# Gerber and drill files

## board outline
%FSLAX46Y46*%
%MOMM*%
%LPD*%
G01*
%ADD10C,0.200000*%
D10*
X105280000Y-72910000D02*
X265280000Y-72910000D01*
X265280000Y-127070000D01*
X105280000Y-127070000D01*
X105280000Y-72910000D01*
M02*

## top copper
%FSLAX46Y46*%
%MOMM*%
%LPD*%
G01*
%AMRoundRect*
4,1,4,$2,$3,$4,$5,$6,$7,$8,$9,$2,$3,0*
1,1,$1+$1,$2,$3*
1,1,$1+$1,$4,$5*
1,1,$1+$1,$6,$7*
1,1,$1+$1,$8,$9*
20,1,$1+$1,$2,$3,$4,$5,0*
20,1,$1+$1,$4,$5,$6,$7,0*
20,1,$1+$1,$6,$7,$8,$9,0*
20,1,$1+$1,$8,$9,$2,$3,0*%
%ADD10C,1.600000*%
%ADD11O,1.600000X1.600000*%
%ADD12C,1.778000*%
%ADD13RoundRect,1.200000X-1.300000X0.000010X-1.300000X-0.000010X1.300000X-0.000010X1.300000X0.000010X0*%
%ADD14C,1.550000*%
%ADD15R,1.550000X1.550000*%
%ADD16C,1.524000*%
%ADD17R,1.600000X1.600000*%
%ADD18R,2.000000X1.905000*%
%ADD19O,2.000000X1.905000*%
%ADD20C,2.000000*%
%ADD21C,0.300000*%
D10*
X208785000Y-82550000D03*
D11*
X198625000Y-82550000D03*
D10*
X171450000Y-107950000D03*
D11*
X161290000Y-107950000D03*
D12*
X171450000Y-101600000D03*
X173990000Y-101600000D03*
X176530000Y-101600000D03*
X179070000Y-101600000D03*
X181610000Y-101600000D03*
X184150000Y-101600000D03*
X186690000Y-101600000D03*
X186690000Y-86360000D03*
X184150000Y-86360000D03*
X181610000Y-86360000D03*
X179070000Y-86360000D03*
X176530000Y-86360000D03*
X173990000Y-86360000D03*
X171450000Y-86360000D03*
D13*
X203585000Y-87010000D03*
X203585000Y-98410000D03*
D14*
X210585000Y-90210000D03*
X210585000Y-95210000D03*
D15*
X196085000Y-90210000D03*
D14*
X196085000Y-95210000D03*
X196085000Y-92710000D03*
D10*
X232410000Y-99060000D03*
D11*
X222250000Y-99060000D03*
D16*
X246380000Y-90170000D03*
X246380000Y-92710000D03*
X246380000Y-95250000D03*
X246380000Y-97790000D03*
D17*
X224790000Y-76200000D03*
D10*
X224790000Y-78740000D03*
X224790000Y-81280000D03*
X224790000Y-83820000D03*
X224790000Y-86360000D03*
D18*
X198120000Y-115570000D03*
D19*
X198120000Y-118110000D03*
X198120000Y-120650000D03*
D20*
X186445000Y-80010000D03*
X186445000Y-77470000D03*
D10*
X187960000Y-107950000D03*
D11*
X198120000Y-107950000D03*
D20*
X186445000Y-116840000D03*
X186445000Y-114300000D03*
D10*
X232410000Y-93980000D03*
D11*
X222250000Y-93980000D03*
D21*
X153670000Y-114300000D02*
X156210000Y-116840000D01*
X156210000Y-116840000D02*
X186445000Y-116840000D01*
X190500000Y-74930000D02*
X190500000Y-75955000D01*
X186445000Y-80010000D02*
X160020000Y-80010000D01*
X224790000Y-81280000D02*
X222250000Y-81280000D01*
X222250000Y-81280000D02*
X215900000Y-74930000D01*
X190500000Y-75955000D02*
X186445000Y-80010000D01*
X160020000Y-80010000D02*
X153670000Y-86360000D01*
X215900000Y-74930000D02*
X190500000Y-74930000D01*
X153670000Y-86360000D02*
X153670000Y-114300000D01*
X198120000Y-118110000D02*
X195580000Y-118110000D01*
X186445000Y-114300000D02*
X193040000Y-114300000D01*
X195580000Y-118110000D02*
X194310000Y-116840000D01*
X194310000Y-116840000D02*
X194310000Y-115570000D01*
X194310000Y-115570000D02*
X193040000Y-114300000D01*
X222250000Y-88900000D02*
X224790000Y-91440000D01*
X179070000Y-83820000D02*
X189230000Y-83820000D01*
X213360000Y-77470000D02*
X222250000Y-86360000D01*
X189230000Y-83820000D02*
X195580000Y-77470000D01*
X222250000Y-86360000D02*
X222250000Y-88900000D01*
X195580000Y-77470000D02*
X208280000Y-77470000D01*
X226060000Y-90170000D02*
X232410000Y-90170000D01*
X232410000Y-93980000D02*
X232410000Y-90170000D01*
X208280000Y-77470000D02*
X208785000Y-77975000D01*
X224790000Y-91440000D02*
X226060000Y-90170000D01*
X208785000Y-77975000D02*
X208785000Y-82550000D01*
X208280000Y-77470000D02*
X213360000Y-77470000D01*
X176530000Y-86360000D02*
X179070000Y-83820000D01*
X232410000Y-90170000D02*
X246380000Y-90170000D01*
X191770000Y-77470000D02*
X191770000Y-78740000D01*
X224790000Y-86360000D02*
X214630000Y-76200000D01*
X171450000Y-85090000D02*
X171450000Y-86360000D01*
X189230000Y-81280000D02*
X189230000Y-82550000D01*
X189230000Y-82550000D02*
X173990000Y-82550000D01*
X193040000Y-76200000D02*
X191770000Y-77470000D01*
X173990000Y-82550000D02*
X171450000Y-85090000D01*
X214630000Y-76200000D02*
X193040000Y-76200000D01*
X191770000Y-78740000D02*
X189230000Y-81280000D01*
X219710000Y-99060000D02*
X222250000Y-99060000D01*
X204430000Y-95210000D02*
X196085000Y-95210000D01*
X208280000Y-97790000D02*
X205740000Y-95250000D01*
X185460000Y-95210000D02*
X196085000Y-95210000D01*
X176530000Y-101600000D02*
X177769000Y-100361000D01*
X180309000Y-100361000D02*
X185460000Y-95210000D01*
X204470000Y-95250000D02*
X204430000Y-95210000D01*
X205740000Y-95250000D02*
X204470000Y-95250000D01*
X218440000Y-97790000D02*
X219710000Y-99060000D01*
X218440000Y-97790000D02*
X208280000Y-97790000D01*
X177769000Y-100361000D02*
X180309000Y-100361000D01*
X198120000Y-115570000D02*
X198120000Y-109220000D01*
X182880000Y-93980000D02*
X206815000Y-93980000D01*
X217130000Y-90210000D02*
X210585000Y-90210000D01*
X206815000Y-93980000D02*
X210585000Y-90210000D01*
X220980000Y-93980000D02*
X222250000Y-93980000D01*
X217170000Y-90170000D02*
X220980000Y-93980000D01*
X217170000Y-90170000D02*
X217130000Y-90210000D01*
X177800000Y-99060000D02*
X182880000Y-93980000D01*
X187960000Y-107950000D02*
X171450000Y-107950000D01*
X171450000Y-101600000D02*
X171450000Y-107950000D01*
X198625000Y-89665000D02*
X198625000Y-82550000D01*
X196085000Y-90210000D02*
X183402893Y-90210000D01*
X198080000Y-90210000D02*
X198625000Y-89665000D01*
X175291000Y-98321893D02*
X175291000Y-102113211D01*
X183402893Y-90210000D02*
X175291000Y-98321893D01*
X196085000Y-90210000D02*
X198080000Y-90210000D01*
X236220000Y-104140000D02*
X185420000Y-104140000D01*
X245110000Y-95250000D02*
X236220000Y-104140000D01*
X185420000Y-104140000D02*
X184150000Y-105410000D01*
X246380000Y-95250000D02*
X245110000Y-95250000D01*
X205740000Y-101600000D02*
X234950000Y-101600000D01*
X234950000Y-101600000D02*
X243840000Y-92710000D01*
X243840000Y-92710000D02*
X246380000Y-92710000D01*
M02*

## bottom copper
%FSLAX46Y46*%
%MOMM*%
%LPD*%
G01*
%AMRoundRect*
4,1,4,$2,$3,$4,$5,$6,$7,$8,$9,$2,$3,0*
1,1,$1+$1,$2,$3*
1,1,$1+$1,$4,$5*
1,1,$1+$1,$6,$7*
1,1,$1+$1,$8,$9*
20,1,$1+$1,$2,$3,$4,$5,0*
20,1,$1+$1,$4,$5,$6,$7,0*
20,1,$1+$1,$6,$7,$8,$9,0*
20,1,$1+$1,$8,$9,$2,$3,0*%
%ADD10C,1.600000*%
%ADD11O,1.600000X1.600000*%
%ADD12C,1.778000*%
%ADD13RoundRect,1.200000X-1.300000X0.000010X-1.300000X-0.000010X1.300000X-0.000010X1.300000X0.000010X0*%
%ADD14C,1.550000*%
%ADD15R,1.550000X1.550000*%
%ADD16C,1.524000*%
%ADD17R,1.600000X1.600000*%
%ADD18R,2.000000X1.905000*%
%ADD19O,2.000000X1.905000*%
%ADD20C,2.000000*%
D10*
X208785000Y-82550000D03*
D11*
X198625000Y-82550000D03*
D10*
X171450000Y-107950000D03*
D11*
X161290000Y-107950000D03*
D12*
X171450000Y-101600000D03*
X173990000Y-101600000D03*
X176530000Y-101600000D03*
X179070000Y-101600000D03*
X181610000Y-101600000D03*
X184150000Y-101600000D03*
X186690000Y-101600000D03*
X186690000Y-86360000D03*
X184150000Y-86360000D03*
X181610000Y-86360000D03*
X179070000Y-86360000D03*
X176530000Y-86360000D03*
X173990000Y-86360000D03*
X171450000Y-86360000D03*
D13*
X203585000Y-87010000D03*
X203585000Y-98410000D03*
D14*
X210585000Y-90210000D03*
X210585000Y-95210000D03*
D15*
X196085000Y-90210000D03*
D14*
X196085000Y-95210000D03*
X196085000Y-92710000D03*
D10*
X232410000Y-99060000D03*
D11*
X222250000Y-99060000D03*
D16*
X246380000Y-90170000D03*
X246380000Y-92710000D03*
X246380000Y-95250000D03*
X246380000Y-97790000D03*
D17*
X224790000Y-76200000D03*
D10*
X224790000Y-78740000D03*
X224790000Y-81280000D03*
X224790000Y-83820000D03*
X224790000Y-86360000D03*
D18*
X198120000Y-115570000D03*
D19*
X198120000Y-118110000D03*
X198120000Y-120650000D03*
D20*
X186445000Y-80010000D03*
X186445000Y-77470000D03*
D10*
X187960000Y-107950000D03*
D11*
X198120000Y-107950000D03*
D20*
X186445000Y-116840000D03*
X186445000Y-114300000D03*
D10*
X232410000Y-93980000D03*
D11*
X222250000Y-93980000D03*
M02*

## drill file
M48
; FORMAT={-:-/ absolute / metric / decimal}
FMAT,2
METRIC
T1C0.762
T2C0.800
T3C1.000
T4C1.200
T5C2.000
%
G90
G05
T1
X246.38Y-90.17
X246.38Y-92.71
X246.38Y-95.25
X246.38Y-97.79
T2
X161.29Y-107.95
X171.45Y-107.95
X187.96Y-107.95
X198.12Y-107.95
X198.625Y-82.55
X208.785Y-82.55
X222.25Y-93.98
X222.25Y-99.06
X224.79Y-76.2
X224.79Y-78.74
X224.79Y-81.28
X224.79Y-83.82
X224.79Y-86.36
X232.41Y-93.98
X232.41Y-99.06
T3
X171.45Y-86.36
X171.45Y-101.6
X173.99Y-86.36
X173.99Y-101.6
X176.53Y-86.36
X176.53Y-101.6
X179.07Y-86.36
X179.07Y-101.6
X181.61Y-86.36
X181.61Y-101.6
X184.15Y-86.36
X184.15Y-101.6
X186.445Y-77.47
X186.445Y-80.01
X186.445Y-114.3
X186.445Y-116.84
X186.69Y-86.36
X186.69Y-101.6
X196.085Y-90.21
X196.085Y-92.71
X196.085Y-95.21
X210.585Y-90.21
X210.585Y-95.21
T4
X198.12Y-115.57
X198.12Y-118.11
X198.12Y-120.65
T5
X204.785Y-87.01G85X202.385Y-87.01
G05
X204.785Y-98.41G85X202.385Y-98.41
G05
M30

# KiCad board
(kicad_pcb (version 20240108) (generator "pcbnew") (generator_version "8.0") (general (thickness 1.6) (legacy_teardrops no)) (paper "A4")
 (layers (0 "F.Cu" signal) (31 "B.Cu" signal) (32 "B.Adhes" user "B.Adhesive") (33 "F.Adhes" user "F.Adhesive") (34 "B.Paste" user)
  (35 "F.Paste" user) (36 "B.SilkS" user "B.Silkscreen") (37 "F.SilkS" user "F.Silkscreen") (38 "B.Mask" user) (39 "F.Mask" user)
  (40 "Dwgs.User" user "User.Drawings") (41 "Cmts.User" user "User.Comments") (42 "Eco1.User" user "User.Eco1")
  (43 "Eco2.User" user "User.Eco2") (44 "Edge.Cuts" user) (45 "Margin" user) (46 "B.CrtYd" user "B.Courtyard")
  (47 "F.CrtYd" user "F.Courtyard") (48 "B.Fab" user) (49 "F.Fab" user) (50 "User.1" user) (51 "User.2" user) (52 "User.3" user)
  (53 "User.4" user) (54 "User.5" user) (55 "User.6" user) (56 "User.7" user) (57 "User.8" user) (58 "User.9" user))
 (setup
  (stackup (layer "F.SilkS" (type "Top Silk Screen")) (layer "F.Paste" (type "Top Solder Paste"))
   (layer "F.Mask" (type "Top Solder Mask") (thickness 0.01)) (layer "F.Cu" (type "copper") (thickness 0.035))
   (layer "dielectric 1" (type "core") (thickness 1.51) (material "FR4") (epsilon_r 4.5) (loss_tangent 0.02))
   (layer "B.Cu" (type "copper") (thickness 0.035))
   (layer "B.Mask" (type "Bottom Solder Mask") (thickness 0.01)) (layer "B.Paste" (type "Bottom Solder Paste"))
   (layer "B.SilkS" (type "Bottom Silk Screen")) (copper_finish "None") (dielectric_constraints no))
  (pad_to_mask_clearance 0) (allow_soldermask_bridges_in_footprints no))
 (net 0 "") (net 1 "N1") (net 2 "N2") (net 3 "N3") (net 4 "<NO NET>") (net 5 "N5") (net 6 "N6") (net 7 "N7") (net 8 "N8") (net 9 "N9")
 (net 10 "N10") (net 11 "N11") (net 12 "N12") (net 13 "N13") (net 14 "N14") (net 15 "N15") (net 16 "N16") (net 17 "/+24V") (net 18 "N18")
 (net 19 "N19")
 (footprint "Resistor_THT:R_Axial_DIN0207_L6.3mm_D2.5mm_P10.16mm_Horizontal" (layer "F.Cu") (at 208.785 82.55 180)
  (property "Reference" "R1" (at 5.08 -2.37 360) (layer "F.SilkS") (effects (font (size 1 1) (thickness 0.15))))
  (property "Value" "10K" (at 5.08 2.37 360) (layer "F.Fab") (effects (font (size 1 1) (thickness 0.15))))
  (pad "1" thru_hole circle (at 0 0 180) (size 1.6 1.6) (drill 0.8) (layers "*.Cu" "*.Mask") (remove_unused_layers no) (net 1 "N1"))
  (pad "2" thru_hole oval (at 10.16 0 180) (size 1.6 1.6) (drill 0.8) (layers "*.Cu" "*.Mask") (remove_unused_layers no) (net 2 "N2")))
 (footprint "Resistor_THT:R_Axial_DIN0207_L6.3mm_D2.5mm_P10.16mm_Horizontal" (layer "F.Cu") (at 171.45 107.95 180)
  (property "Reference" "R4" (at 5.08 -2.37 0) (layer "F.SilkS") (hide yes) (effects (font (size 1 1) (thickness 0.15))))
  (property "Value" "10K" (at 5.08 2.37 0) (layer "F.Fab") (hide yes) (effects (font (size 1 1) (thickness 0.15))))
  (pad "1" thru_hole circle (at 0 0 180) (size 1.6 1.6) (drill 0.8) (layers "*.Cu" "*.Mask") (remove_unused_layers no) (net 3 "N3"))
  (pad "2" thru_hole oval (at 10.16 0 180) (size 1.6 1.6) (drill 0.8) (layers "*.Cu" "*.Mask") (remove_unused_layers no) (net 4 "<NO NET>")))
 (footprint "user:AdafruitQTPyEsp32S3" (layer "F.Cu") (at 171.45 101.6 90)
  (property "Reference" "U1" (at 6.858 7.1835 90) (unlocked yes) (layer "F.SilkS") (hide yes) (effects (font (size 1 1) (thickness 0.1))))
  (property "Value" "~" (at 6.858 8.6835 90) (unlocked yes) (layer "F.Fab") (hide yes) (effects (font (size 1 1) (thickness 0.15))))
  (pad "1" thru_hole circle (at 0 0 90) (size 1.778 1.778) (drill 1) (layers "*.Cu" "*.Mask") (remove_unused_layers no) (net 3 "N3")
   (solder_mask_margin 0.0508) (thermal_bridge_angle 0))
  (pad "2" thru_hole circle (at 0 2.54 90) (size 1.778 1.778) (drill 1) (layers "*.Cu" "*.Mask") (remove_unused_layers no) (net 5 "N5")
   (solder_mask_margin 0.0508) (thermal_bridge_angle 0))
  (pad "3" thru_hole circle (at 0 5.08 90) (size 1.778 1.778) (drill 1) (layers "*.Cu" "*.Mask") (remove_unused_layers no) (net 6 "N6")
   (solder_mask_margin 0.0508) (thermal_bridge_angle 0))
  (pad "4" thru_hole circle (at 0 7.62 90) (size 1.778 1.778) (drill 1) (layers "*.Cu" "*.Mask") (remove_unused_layers no) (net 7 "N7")
   (solder_mask_margin 0.0508) (thermal_bridge_angle 0))
  (pad "5" thru_hole circle (at 0 10.16 90) (size 1.778 1.778) (drill 1) (layers "*.Cu" "*.Mask") (remove_unused_layers no) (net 2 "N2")
   (solder_mask_margin 0.0508) (thermal_bridge_angle 0))
  (pad "6" thru_hole circle (at 0 12.7 90) (size 1.778 1.778) (drill 1) (layers "*.Cu" "*.Mask") (remove_unused_layers no) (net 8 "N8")
   (solder_mask_margin 0.0508) (thermal_bridge_angle 0))
  (pad "7" thru_hole circle (at 0 15.24 90) (size 1.778 1.778) (drill 1) (layers "*.Cu" "*.Mask") (remove_unused_layers no) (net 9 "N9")
   (solder_mask_margin 0.0508) (thermal_bridge_angle 0))
  (pad "8" thru_hole circle (at 15.24 15.24 270) (size 1.778 1.778) (drill 1) (layers "*.Cu" "*.Mask") (remove_unused_layers no)
   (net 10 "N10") (solder_mask_margin 0.0508) (thermal_bridge_angle 0))
  (pad "9" thru_hole circle (at 15.24 12.7 270) (size 1.778 1.778) (drill 1) (layers "*.Cu" "*.Mask") (remove_unused_layers no)
   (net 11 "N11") (solder_mask_margin 0.0508) (thermal_bridge_angle 0))
  (pad "10" thru_hole circle (at 15.24 10.16 270) (size 1.778 1.778) (drill 1) (layers "*.Cu" "*.Mask") (remove_unused_layers no)
   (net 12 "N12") (solder_mask_margin 0.0508) (thermal_bridge_angle 0))
  (pad "11" thru_hole circle (at 15.24 7.62 270) (size 1.778 1.778) (drill 1) (layers "*.Cu" "*.Mask") (remove_unused_layers no)
   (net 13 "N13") (solder_mask_margin 0.0508) (thermal_bridge_angle 0))
  (pad "12" thru_hole circle (at 15.24 5.08 270) (size 1.778 1.778) (drill 1) (layers "*.Cu" "*.Mask") (remove_unused_layers no)
   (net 1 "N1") (solder_mask_margin 0.0508) (thermal_bridge_angle 0))
  (pad "13" thru_hole circle (at 15.24 2.54 270) (size 1.778 1.778) (drill 1) (layers "*.Cu" "*.Mask") (remove_unused_layers no)
   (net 4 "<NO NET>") (solder_mask_margin 0.0508) (thermal_bridge_angle 0))
  (pad "14" thru_hole circle (at 15.24 0 270) (size 1.778 1.778) (drill 1) (layers "*.Cu" "*.Mask") (remove_unused_layers no) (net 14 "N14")
   (solder_mask_margin 0.0508) (thermal_bridge_angle 0)))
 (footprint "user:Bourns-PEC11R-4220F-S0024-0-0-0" (layer "F.Cu") (at 203.585 92.71 -90)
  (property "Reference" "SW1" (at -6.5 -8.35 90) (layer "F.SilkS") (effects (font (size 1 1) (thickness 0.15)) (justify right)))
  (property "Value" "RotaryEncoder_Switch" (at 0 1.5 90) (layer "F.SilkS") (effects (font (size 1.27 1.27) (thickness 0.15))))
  (pad "" thru_hole roundrect (at -5.7 0 270) (size 2.4 5) (drill oval 2 4.4) (layers "*.Cu" "*.Mask") (remove_unused_layers no)
   (roundrect_rratio 0.5))
  (pad "" thru_hole roundrect (at 5.7 0 270) (size 2.4 5) (drill oval 2 4.4) (layers "*.Cu" "*.Mask") (remove_unused_layers no)
   (roundrect_rratio 0.5))
  (pad "1" thru_hole circle (at -2.5 -7 270) (size 1.55 1.55) (drill 1) (layers "*.Cu" "*.Mask") (remove_unused_layers no) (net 12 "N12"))
  (pad "2" thru_hole circle (at 2.5 -7 270) (size 1.55 1.55) (drill 1) (layers "*.Cu" "*.Mask") (remove_unused_layers no) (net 4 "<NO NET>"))
  (pad "A" thru_hole rect (at -2.5 7.5 270) (size 1.55 1.55) (drill 1) (layers "*.Cu" "*.Mask") (remove_unused_layers no) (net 2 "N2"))
  (pad "B" thru_hole circle (at 2.5 7.5 270) (size 1.55 1.55) (drill 1) (layers "*.Cu" "*.Mask") (remove_unused_layers no) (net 6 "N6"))
  (pad "C" thru_hole circle (at 0 7.5 270) (size 1.55 1.55) (drill 1) (layers "*.Cu" "*.Mask") (remove_unused_layers no) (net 4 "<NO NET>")))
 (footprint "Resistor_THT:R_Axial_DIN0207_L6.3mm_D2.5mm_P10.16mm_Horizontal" (layer "F.Cu") (at 232.41 99.06 180)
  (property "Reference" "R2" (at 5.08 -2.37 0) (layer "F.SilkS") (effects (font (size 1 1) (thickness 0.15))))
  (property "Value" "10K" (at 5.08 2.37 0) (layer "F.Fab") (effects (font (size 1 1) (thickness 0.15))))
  (pad "1" thru_hole circle (at 0 0 180) (size 1.6 1.6) (drill 0.8) (layers "*.Cu" "*.Mask") (remove_unused_layers no) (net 1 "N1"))
  (pad "2" thru_hole oval (at 10.16 0 180) (size 1.6 1.6) (drill 0.8) (layers "*.Cu" "*.Mask") (remove_unused_layers no) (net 6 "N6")))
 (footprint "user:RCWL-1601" (layer "F.Cu") (at 246.38 90.17 -90)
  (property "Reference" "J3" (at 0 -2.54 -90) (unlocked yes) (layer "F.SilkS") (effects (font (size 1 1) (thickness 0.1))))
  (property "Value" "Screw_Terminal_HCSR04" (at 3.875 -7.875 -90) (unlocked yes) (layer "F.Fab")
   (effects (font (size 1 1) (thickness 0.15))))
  (pad "1" thru_hole circle (at 0 0 270) (size 1.524 1.524) (drill 0.762) (layers "*.Cu" "*.Mask") (remove_unused_layers no) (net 1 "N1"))
  (pad "2" thru_hole circle (at 2.54 0 270) (size 1.524 1.524) (drill 0.762) (layers "*.Cu" "*.Mask") (remove_unused_layers no)
   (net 10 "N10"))
  (pad "3" thru_hole circle (at 5.08 0 270) (size 1.524 1.524) (drill 0.762) (layers "*.Cu" "*.Mask") (remove_unused_layers no) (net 9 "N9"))
  (pad "4" thru_hole circle (at 7.62 0 270) (size 1.524 1.524) (drill 0.762) (layers "*.Cu" "*.Mask") (remove_unused_layers no)
   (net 4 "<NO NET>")))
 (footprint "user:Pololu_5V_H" (layer "F.Cu") (at 224.79 81.28 -90)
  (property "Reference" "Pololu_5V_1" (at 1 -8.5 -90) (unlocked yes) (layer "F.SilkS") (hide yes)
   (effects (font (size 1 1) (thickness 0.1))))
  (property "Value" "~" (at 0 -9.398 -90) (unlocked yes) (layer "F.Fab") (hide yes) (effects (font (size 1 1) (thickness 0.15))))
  (pad "1" thru_hole rect (at -5.08 0 270) (size 1.6 1.6) (drill 0.8) (layers "*.Cu" "*.Mask") (remove_unused_layers no) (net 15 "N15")
   (thermal_bridge_angle 45))
  (pad "2" thru_hole circle (at -2.54 0 270) (size 1.6 1.6) (drill 0.8) (layers "*.Cu" "*.Mask") (remove_unused_layers no) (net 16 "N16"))
  (pad "3" thru_hole circle (at 0 0 270) (size 1.6 1.6) (drill 0.8) (layers "*.Cu" "*.Mask") (remove_unused_layers no) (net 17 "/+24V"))
  (pad "4" thru_hole circle (at 2.54 0 270) (size 1.6 1.6) (drill 0.8) (layers "*.Cu" "*.Mask") (remove_unused_layers no) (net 4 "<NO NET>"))
  (pad "5" thru_hole circle (at 5.08 0 270) (size 1.6 1.6) (drill 0.8) (layers "*.Cu" "*.Mask") (remove_unused_layers no) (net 14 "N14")))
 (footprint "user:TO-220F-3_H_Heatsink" (layer "F.Cu") (at 198.12 115.57 -90)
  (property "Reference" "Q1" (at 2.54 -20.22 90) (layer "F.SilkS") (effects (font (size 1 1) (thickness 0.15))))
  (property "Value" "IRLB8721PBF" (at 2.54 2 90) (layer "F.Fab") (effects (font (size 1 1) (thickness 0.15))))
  (pad "1" thru_hole rect (at 0 0 270) (size 1.905 2) (drill 1.2) (layers "*.Cu" "*.Mask") (remove_unused_layers no) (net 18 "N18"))
  (pad "2" thru_hole oval (at 2.54 0 270) (size 1.905 2) (drill 1.2) (layers "*.Cu" "*.Mask") (remove_unused_layers no) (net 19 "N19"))
  (pad "3" thru_hole oval (at 5.08 0 270) (size 1.905 2) (drill 1.2) (layers "*.Cu" "*.Mask") (remove_unused_layers no) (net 4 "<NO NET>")))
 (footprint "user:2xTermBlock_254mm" (layer "F.Cu") (at 186.445 80.01 90)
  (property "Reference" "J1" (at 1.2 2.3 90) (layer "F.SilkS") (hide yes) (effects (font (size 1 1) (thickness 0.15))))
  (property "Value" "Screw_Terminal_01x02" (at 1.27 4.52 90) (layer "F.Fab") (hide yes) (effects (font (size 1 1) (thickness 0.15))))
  (pad "1" thru_hole circle (at 0 0 90) (size 2 2) (drill 1) (layers "*.Cu" "*.Mask") (remove_unused_layers no) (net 17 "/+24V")
   (thermal_bridge_angle 90))
  (pad "2" thru_hole circle (at 2.54 0 90) (size 2 2) (drill 1) (layers "*.Cu" "*.Mask") (remove_unused_layers no) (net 4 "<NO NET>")))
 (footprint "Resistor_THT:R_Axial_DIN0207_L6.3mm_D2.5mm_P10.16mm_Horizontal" (layer "F.Cu") (at 187.96 107.95)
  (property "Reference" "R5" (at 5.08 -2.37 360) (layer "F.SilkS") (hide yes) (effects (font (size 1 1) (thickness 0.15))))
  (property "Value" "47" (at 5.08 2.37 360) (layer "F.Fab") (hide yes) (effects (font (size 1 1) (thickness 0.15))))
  (pad "1" thru_hole circle (at 0 0) (size 1.6 1.6) (drill 0.8) (layers "*.Cu" "*.Mask") (remove_unused_layers no) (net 3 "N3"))
  (pad "2" thru_hole oval (at 10.16 0) (size 1.6 1.6) (drill 0.8) (layers "*.Cu" "*.Mask") (remove_unused_layers no) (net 18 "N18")))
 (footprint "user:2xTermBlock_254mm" (layer "F.Cu") (at 186.445 116.84 90)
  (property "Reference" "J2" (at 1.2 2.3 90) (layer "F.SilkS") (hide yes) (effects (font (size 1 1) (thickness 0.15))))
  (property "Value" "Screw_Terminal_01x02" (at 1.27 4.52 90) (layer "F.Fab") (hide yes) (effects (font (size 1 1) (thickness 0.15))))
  (pad "1" thru_hole circle (at 0 0 90) (size 2 2) (drill 1) (layers "*.Cu" "*.Mask") (remove_unused_layers no) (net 17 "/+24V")
   (thermal_bridge_angle 90))
  (pad "2" thru_hole circle (at 2.54 0 90) (size 2 2) (drill 1) (layers "*.Cu" "*.Mask") (remove_unused_layers no) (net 19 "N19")))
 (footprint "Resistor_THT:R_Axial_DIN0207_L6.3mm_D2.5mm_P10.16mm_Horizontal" (layer "F.Cu") (at 232.41 93.98 180)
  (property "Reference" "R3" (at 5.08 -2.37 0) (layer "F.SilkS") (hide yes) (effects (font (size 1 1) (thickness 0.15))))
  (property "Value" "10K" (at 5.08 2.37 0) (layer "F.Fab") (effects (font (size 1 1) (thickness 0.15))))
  (pad "1" thru_hole circle (at 0 0 180) (size 1.6 1.6) (drill 0.8) (layers "*.Cu" "*.Mask") (remove_unused_layers no) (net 1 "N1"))
  (pad "2" thru_hole oval (at 10.16 0 180) (size 1.6 1.6) (drill 0.8) (layers "*.Cu" "*.Mask") (remove_unused_layers no) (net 12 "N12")))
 (gr_rect (start 105.28 72.91) (end 265.28 127.07) (stroke (width 0.2) (type default)) (fill none) (layer "Edge.Cuts"))
 (segment (start 153.67 114.3) (end 156.21 116.84) (width 0.3) (layer "F.Cu") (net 17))
 (segment (start 156.21 116.84) (end 186.445 116.84) (width 0.3) (layer "F.Cu") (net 17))
 (segment (start 190.5 74.93) (end 190.5 75.955) (width 0.3) (layer "F.Cu") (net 17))
 (segment (start 186.445 80.01) (end 160.02 80.01) (width 0.3) (layer "F.Cu") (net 17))
 (segment (start 224.79 81.28) (end 222.25 81.28) (width 0.3) (layer "F.Cu") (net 17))
 (segment (start 222.25 81.28) (end 215.9 74.93) (width 0.3) (layer "F.Cu") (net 17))
 (segment (start 190.5 75.955) (end 186.445 80.01) (width 0.3) (layer "F.Cu") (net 17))
 (segment (start 160.02 80.01) (end 153.67 86.36) (width 0.3) (layer "F.Cu") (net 17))
 (segment (start 215.9 74.93) (end 190.5 74.93) (width 0.3) (layer "F.Cu") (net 17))
 (segment (start 153.67 86.36) (end 153.67 114.3) (width 0.3) (layer "F.Cu") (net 17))
 (segment (start 198.12 118.11) (end 195.58 118.11) (width 0.3) (layer "F.Cu") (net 19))
 (segment (start 186.445 114.3) (end 193.04 114.3) (width 0.3) (layer "F.Cu") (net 19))
 (segment (start 195.58 118.11) (end 194.31 116.84) (width 0.3) (layer "F.Cu") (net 19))
 (segment (start 194.31 116.84) (end 194.31 115.57) (width 0.3) (layer "F.Cu") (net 19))
 (segment (start 194.31 115.57) (end 193.04 114.3) (width 0.3) (layer "F.Cu") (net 19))
 (segment (start 222.25 88.9) (end 224.79 91.44) (width 0.3) (layer "F.Cu") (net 1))
 (segment (start 179.07 83.82) (end 189.23 83.82) (width 0.3) (layer "F.Cu") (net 1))
 (segment (start 213.36 77.47) (end 222.25 86.36) (width 0.3) (layer "F.Cu") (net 1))
 (segment (start 189.23 83.82) (end 195.58 77.47) (width 0.3) (layer "F.Cu") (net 1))
 (segment (start 222.25 86.36) (end 222.25 88.9) (width 0.3) (layer "F.Cu") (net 1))
 (segment (start 195.58 77.47) (end 208.28 77.47) (width 0.3) (layer "F.Cu") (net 1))
 (segment (start 226.06 90.17) (end 232.41 90.17) (width 0.3) (layer "F.Cu") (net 1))
 (segment (start 232.41 93.98) (end 232.41 90.17) (width 0.3) (layer "F.Cu") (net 1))
 (segment (start 208.28 77.47) (end 208.785 77.975) (width 0.3) (layer "F.Cu") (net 1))
 (segment (start 224.79 91.44) (end 226.06 90.17) (width 0.3) (layer "F.Cu") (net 1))
 (segment (start 208.785 77.975) (end 208.785 82.55) (width 0.3) (layer "F.Cu") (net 1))
 (segment (start 208.28 77.47) (end 213.36 77.47) (width 0.3) (layer "F.Cu") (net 1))
 (segment (start 176.53 86.36) (end 179.07 83.82) (width 0.3) (layer "F.Cu") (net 1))
 (segment (start 232.41 90.17) (end 246.38 90.17) (width 0.3) (layer "F.Cu") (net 1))
 (segment (start 191.77 77.47) (end 191.77 78.74) (width 0.3) (layer "F.Cu") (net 14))
 (segment (start 224.79 86.36) (end 214.63 76.2) (width 0.3) (layer "F.Cu") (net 14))
 (segment (start 171.45 85.09) (end 171.45 86.36) (width 0.3) (layer "F.Cu") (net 14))
 (segment (start 189.23 81.28) (end 189.23 82.55) (width 0.3) (layer "F.Cu") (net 14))
 (segment (start 189.23 82.55) (end 173.99 82.55) (width 0.3) (layer "F.Cu") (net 14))
 (segment (start 193.04 76.2) (end 191.77 77.47) (width 0.3) (layer "F.Cu") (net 14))
 (segment (start 173.99 82.55) (end 171.45 85.09) (width 0.3) (layer "F.Cu") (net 14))
 (segment (start 214.63 76.2) (end 193.04 76.2) (width 0.3) (layer "F.Cu") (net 14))
 (segment (start 191.77 78.74) (end 189.23 81.28) (width 0.3) (layer "F.Cu") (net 14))
 (segment (start 219.71 99.06) (end 222.25 99.06) (width 0.3) (layer "F.Cu") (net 6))
 (segment (start 204.43 95.21) (end 196.085 95.21) (width 0.3) (layer "F.Cu") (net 6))
 (segment (start 208.28 97.79) (end 205.74 95.25) (width 0.3) (layer "F.Cu") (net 6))
 (segment (start 185.46 95.21) (end 196.085 95.21) (width 0.3) (layer "F.Cu") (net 6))
 (segment (start 176.53 101.6) (end 177.769 100.361) (width 0.3) (layer "F.Cu") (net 6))
 (segment (start 180.309 100.361) (end 185.46 95.21) (width 0.3) (layer "F.Cu") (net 6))
 (segment (start 204.47 95.25) (end 204.43 95.21) (width 0.3) (layer "F.Cu") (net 6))
 (segment (start 205.74 95.25) (end 204.47 95.25) (width 0.3) (layer "F.Cu") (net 6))
 (segment (start 218.44 97.79) (end 219.71 99.06) (width 0.3) (layer "F.Cu") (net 6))
 (segment (start 218.44 97.79) (end 208.28 97.79) (width 0.3) (layer "F.Cu") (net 6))
 (segment (start 177.769 100.361) (end 180.309 100.361) (width 0.3) (layer "F.Cu") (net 6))
 (segment (start 198.12 115.57) (end 198.12 109.22) (width 0.3) (layer "F.Cu") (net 18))
 (segment (start 182.88 93.98) (end 206.815 93.98) (width 0.3) (layer "F.Cu") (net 12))
 (segment (start 217.13 90.21) (end 210.585 90.21) (width 0.3) (layer "F.Cu") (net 12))
 (segment (start 206.815 93.98) (end 210.585 90.21) (width 0.3) (layer "F.Cu") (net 12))
 (segment (start 220.98 93.98) (end 222.25 93.98) (width 0.3) (layer "F.Cu") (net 12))
 (segment (start 217.17 90.17) (end 220.98 93.98) (width 0.3) (layer "F.Cu") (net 12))
 (segment (start 217.17 90.17) (end 217.13 90.21) (width 0.3) (layer "F.Cu") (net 12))
 (segment (start 177.8 99.06) (end 182.88 93.98) (width 0.3) (layer "F.Cu") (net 12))
 (segment (start 187.96 107.95) (end 171.45 107.95) (width 0.3) (layer "F.Cu") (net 3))
 (segment (start 171.45 101.6) (end 171.45 107.95) (width 0.3) (layer "F.Cu") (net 3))
 (segment (start 198.625 89.665) (end 198.625 82.55) (width 0.3) (layer "F.Cu") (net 2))
 (segment (start 196.085 90.21) (end 183.402893 90.21) (width 0.3) (layer "F.Cu") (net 2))
 (segment (start 198.08 90.21) (end 198.625 89.665) (width 0.3) (layer "F.Cu") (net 2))
 (segment (start 175.291 98.321893) (end 175.291 102.113211) (width 0.3) (layer "F.Cu") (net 2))
 (segment (start 183.402893 90.21) (end 175.291 98.321893) (width 0.3) (layer "F.Cu") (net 2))
 (segment (start 196.085 90.21) (end 198.08 90.21) (width 0.3) (layer "F.Cu") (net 2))
 (segment (start 236.22 104.14) (end 185.42 104.14) (width 0.3) (layer "F.Cu") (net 9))
 (segment (start 245.11 95.25) (end 236.22 104.14) (width 0.3) (layer "F.Cu") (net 9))
 (segment (start 185.42 104.14) (end 184.15 105.41) (width 0.3) (layer "F.Cu") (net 9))
 (segment (start 246.38 95.25) (end 245.11 95.25) (width 0.3) (layer "F.Cu") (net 9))
 (segment (start 205.74 101.6) (end 234.95 101.6) (width 0.3) (layer "F.Cu") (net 10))
 (segment (start 234.95 101.6) (end 243.84 92.71) (width 0.3) (layer "F.Cu") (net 10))
 (segment (start 243.84 92.71) (end 246.38 92.71) (width 0.3) (layer "F.Cu") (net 10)))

